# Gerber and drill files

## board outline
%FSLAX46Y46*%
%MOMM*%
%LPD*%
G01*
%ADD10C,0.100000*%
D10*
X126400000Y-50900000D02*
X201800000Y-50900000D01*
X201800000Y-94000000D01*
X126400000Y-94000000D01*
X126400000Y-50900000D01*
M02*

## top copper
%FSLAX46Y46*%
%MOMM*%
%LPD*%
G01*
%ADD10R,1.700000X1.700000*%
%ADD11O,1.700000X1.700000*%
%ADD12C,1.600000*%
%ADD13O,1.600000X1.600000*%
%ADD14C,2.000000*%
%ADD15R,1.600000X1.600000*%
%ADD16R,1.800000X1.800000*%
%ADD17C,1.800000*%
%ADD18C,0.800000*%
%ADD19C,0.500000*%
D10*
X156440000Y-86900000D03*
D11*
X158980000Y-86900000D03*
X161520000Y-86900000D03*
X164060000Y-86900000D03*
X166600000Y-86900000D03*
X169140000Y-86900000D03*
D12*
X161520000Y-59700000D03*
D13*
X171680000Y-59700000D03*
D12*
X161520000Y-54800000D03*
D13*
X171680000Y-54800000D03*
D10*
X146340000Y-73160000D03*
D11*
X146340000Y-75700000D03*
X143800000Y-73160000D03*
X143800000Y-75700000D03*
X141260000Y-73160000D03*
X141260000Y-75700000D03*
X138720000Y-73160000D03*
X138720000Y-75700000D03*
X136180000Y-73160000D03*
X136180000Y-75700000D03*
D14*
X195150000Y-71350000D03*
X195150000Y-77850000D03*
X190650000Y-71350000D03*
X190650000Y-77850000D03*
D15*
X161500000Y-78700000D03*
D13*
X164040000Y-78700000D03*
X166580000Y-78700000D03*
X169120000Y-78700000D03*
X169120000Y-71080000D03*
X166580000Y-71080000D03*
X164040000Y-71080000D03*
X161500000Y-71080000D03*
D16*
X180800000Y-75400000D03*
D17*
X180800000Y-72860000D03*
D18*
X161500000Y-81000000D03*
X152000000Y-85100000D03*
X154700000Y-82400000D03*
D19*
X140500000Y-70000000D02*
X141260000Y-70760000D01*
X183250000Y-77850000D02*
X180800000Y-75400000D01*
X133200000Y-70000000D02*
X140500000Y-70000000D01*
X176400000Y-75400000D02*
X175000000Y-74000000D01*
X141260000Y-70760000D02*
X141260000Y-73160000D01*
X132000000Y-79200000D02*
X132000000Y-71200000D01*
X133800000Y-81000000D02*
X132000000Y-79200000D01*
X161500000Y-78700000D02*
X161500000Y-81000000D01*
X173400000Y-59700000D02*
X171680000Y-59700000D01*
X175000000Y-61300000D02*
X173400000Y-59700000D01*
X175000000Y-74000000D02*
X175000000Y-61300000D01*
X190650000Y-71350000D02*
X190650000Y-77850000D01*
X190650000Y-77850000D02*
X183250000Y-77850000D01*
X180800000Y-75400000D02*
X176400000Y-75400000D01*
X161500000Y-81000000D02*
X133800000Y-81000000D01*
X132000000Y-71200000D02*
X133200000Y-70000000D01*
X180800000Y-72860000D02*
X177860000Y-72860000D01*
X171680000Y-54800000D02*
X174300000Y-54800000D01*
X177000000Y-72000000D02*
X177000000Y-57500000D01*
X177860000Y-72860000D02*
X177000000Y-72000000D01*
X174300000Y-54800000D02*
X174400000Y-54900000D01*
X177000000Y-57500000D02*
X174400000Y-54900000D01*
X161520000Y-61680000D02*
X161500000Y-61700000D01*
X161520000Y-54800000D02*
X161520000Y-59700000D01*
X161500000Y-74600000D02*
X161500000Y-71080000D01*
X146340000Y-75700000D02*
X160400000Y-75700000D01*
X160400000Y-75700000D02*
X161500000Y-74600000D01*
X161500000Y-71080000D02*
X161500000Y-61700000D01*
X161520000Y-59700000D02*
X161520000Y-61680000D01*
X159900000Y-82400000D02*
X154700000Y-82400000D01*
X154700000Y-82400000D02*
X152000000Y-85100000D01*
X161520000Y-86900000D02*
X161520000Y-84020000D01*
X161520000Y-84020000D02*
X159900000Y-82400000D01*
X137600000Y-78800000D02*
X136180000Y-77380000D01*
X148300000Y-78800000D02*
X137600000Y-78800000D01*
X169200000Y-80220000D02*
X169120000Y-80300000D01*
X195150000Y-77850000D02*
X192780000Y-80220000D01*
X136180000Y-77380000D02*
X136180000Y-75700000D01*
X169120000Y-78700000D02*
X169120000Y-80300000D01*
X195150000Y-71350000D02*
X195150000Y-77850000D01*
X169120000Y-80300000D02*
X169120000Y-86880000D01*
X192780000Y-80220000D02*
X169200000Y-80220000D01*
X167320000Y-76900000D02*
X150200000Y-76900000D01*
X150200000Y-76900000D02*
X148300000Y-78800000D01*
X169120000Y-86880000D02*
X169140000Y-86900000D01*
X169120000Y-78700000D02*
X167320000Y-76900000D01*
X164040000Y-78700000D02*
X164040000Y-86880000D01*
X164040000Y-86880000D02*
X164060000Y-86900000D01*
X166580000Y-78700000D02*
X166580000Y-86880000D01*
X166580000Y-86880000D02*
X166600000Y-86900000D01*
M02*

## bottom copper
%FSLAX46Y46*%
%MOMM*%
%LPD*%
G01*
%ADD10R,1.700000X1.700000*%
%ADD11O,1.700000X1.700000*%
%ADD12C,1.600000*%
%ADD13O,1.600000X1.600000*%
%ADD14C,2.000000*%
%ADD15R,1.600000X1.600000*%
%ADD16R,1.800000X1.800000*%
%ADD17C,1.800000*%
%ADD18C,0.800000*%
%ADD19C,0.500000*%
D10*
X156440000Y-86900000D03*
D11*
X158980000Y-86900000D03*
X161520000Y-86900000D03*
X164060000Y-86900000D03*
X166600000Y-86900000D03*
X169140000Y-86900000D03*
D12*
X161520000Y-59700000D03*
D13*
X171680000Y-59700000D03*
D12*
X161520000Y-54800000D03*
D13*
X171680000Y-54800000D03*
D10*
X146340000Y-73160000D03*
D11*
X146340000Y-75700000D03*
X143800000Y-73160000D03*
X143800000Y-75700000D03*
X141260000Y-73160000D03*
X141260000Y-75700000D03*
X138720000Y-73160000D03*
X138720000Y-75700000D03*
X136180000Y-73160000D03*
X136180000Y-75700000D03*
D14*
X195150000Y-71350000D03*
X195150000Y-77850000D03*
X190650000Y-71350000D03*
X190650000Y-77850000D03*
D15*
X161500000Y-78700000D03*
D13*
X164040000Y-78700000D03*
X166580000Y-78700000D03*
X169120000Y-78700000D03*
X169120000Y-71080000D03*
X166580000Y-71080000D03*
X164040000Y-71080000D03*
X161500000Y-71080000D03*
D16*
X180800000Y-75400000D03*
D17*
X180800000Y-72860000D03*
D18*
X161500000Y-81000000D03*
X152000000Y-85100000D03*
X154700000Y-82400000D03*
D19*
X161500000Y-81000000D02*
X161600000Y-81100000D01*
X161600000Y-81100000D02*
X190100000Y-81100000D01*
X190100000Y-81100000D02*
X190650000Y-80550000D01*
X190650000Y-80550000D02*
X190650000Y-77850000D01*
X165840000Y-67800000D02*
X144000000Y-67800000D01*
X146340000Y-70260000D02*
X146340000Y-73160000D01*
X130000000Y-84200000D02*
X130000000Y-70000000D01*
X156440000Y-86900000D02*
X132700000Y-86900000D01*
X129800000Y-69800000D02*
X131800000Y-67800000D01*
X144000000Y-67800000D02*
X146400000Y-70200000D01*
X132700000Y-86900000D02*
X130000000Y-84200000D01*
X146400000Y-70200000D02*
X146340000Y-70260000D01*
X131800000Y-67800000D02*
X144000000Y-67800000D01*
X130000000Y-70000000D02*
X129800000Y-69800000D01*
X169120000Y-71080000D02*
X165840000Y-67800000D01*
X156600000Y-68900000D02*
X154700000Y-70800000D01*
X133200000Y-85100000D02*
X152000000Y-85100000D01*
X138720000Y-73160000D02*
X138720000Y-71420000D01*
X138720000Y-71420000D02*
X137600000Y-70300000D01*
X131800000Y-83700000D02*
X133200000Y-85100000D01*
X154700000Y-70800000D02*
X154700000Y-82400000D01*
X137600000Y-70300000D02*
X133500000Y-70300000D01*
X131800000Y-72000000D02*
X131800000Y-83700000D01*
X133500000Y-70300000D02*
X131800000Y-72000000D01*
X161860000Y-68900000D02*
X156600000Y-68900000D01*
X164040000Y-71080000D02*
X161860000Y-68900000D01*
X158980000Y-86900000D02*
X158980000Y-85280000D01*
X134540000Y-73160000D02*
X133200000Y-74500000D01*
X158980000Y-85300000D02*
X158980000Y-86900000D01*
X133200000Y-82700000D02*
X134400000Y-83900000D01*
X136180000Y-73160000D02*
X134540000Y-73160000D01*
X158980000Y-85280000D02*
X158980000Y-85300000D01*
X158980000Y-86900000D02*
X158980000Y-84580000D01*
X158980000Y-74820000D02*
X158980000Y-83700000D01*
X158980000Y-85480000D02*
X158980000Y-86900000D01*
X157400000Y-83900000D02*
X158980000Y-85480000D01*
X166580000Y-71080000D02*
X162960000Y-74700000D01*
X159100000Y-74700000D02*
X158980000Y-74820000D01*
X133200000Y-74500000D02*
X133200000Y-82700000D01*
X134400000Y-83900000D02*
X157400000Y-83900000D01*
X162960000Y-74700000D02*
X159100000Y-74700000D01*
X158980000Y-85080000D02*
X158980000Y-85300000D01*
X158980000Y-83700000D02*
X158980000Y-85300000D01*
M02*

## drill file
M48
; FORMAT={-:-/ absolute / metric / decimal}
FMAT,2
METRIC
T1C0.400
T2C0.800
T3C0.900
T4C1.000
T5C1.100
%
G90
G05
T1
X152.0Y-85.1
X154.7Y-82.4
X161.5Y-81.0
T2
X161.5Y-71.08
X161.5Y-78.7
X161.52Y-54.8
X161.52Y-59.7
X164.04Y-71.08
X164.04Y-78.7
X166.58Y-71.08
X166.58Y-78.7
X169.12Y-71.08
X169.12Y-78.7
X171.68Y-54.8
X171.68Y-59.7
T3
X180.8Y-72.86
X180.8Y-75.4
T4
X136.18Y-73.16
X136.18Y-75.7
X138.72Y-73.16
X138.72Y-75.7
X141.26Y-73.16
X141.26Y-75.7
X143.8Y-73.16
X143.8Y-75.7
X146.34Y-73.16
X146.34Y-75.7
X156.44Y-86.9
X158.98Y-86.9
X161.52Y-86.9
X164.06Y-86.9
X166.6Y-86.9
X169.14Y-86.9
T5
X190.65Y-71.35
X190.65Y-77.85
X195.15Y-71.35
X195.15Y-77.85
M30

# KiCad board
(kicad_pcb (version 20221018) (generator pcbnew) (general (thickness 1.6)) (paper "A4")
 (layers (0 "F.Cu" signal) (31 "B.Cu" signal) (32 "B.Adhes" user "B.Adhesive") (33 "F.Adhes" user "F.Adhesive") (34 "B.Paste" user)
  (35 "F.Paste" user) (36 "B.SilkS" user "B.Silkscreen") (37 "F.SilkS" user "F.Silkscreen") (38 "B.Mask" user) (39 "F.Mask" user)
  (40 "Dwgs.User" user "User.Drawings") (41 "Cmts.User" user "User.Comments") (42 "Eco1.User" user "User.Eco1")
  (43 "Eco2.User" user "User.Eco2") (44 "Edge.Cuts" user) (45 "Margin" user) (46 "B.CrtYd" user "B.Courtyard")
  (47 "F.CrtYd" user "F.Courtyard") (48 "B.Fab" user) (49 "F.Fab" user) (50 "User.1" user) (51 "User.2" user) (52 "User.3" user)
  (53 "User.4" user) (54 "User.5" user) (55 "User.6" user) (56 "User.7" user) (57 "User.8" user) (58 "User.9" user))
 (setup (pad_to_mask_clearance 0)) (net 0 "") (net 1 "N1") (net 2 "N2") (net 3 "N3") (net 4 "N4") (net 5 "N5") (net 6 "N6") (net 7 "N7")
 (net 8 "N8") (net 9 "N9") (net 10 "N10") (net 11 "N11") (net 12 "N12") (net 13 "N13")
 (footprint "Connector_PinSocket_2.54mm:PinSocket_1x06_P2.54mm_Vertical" (layer "F.Cu") (at 156.44 86.9 90)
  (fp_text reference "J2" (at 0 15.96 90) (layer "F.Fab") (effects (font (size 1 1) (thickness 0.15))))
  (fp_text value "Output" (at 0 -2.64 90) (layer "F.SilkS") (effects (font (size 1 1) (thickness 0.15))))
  (pad "1" thru_hole rect (at 0 0 90) (size 1.7 1.7) (drill 1) (layers "*.Cu" "*.Mask") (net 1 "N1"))
  (pad "2" thru_hole oval (at 0 2.54 90) (size 1.7 1.7) (drill 1) (layers "*.Cu" "*.Mask") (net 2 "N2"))
  (pad "3" thru_hole oval (at 0 5.08 90) (size 1.7 1.7) (drill 1) (layers "*.Cu" "*.Mask") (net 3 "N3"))
  (pad "4" thru_hole oval (at 0 7.62 90) (size 1.7 1.7) (drill 1) (layers "*.Cu" "*.Mask") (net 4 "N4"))
  (pad "5" thru_hole oval (at 0 10.16 90) (size 1.7 1.7) (drill 1) (layers "*.Cu" "*.Mask") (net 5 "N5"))
  (pad "6" thru_hole oval (at 0 12.7 90) (size 1.7 1.7) (drill 1) (layers "*.Cu" "*.Mask") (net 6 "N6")))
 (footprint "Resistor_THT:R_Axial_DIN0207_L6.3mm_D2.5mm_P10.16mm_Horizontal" (layer "F.Cu") (at 161.52 59.7)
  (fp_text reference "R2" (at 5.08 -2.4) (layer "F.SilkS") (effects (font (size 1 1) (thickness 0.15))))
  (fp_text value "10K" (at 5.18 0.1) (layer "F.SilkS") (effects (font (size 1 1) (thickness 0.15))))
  (pad "1" thru_hole circle (at 0 0) (size 1.6 1.6) (drill 0.8) (layers "*.Cu" "*.Mask") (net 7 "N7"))
  (pad "2" thru_hole oval (at 10.16 0) (size 1.6 1.6) (drill 0.8) (layers "*.Cu" "*.Mask") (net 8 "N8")))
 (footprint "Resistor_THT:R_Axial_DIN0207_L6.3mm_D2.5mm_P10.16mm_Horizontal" (layer "F.Cu") (at 161.52 54.8)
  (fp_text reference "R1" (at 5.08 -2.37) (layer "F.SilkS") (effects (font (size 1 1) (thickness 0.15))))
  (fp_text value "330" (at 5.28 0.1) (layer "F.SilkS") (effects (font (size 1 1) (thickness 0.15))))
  (pad "1" thru_hole circle (at 0 0) (size 1.6 1.6) (drill 0.8) (layers "*.Cu" "*.Mask") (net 7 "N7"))
  (pad "2" thru_hole oval (at 10.16 0) (size 1.6 1.6) (drill 0.8) (layers "*.Cu" "*.Mask") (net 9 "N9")))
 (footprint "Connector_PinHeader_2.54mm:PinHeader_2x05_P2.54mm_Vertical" (layer "F.Cu") (at 146.34 73.16 -90)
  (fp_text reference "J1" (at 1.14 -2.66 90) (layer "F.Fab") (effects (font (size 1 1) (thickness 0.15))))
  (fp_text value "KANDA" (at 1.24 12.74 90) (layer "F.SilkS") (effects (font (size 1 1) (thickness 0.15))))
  (pad "1" thru_hole rect (at 0 0 270) (size 1.7 1.7) (drill 1) (layers "*.Cu" "*.Mask") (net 1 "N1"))
  (pad "2" thru_hole oval (at 2.54 0 270) (size 1.7 1.7) (drill 1) (layers "*.Cu" "*.Mask") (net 7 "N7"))
  (pad "3" thru_hole oval (at 0 2.54 270) (size 1.7 1.7) (drill 1) (layers "*.Cu" "*.Mask") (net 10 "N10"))
  (pad "4" thru_hole oval (at 2.54 2.54 270) (size 1.7 1.7) (drill 1) (layers "*.Cu" "*.Mask") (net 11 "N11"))
  (pad "5" thru_hole oval (at 0 5.08 270) (size 1.7 1.7) (drill 1) (layers "*.Cu" "*.Mask") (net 8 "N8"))
  (pad "6" thru_hole oval (at 2.54 5.08 270) (size 1.7 1.7) (drill 1) (layers "*.Cu" "*.Mask") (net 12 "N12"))
  (pad "7" thru_hole oval (at 0 7.62 270) (size 1.7 1.7) (drill 1) (layers "*.Cu" "*.Mask") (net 3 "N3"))
  (pad "8" thru_hole oval (at 2.54 7.62 270) (size 1.7 1.7) (drill 1) (layers "*.Cu" "*.Mask") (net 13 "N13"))
  (pad "9" thru_hole oval (at 0 10.16 270) (size 1.7 1.7) (drill 1) (layers "*.Cu" "*.Mask") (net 2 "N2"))
  (pad "10" thru_hole oval (at 2.54 10.16 270) (size 1.7 1.7) (drill 1) (layers "*.Cu" "*.Mask") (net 6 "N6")))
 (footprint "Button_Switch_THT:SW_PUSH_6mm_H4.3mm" (layer "F.Cu") (at 195.15 71.35 -90)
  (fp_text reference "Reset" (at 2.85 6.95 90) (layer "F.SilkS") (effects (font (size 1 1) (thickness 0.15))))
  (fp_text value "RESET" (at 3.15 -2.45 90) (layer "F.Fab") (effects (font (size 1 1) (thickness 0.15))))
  (pad "1" thru_hole circle (at 0 0) (size 2 2) (drill 1.1) (layers "*.Cu" "*.Mask") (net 6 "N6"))
  (pad "1" thru_hole circle (at 6.5 0) (size 2 2) (drill 1.1) (layers "*.Cu" "*.Mask") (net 6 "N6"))
  (pad "2" thru_hole circle (at 0 4.5) (size 2 2) (drill 1.1) (layers "*.Cu" "*.Mask") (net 8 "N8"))
  (pad "2" thru_hole circle (at 6.5 4.5) (size 2 2) (drill 1.1) (layers "*.Cu" "*.Mask") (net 8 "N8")))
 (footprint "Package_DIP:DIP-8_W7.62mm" (layer "F.Cu") (at 161.5 78.7 90)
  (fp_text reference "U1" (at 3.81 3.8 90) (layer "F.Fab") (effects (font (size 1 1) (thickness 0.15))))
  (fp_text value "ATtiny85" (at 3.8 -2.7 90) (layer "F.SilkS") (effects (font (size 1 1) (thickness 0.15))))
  (pad "1" thru_hole rect (at 0 0 90) (size 1.6 1.6) (drill 0.8) (layers "*.Cu" "*.Mask") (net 8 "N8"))
  (pad "2" thru_hole oval (at 0 2.54 90) (size 1.6 1.6) (drill 0.8) (layers "*.Cu" "*.Mask") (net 4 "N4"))
  (pad "3" thru_hole oval (at 0 5.08 90) (size 1.6 1.6) (drill 0.8) (layers "*.Cu" "*.Mask") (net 5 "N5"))
  (pad "4" thru_hole oval (at 0 7.62 90) (size 1.6 1.6) (drill 0.8) (layers "*.Cu" "*.Mask") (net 6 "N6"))
  (pad "5" thru_hole oval (at 7.62 7.62 90) (size 1.6 1.6) (drill 0.8) (layers "*.Cu" "*.Mask") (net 1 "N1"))
  (pad "6" thru_hole oval (at 7.62 5.08 90) (size 1.6 1.6) (drill 0.8) (layers "*.Cu" "*.Mask") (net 2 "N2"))
  (pad "7" thru_hole oval (at 7.62 2.54 90) (size 1.6 1.6) (drill 0.8) (layers "*.Cu" "*.Mask") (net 3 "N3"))
  (pad "8" thru_hole oval (at 7.62 0 90) (size 1.6 1.6) (drill 0.8) (layers "*.Cu" "*.Mask") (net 7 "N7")))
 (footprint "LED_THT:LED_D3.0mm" (layer "F.Cu") (at 180.8 75.4 90)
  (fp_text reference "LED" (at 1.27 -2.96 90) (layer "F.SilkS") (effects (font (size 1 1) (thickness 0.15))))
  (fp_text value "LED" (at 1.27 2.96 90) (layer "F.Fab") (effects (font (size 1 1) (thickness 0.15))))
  (pad "1" thru_hole rect (at 0 0 90) (size 1.8 1.8) (drill 0.9) (layers "*.Cu" "*.Mask") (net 8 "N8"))
  (pad "2" thru_hole circle (at 2.54 0 90) (size 1.8 1.8) (drill 0.9) (layers "*.Cu" "*.Mask") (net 9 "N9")))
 (gr_rect (start 126.4 50.9) (end 201.8 94) (stroke (width 0.1) (type default)) (fill none) (layer "Edge.Cuts"))
 (segment (start 140.5 70) (end 141.26 70.76) (width 0.5) (layer "F.Cu") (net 8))
 (segment (start 183.25 77.85) (end 180.8 75.4) (width 0.5) (layer "F.Cu") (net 8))
 (segment (start 133.2 70) (end 140.5 70) (width 0.5) (layer "F.Cu") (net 8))
 (segment (start 176.4 75.4) (end 175 74) (width 0.5) (layer "F.Cu") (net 8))
 (segment (start 141.26 70.76) (end 141.26 73.16) (width 0.5) (layer "F.Cu") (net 8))
 (segment (start 132 79.2) (end 132 71.2) (width 0.5) (layer "F.Cu") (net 8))
 (segment (start 133.8 81) (end 132 79.2) (width 0.5) (layer "F.Cu") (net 8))
 (segment (start 161.5 78.7) (end 161.5 81) (width 0.5) (layer "F.Cu") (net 8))
 (segment (start 173.4 59.7) (end 171.68 59.7) (width 0.5) (layer "F.Cu") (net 8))
 (segment (start 175 61.3) (end 173.4 59.7) (width 0.5) (layer "F.Cu") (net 8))
 (segment (start 175 74) (end 175 61.3) (width 0.5) (layer "F.Cu") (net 8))
 (segment (start 190.65 71.35) (end 190.65 77.85) (width 0.5) (layer "F.Cu") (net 8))
 (segment (start 190.65 77.85) (end 183.25 77.85) (width 0.5) (layer "F.Cu") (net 8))
 (segment (start 180.8 75.4) (end 176.4 75.4) (width 0.5) (layer "F.Cu") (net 8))
 (segment (start 161.5 81) (end 133.8 81) (width 0.5) (layer "F.Cu") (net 8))
 (segment (start 132 71.2) (end 133.2 70) (width 0.5) (layer "F.Cu") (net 8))
 (via (at 161.5 81) (size 0.8) (drill 0.4) (layers "F.Cu" "B.Cu") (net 8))
 (segment (start 161.5 81) (end 161.6 81.1) (width 0.5) (layer "B.Cu") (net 8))
 (segment (start 161.6 81.1) (end 190.1 81.1) (width 0.5) (layer "B.Cu") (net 8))
 (segment (start 190.1 81.1) (end 190.65 80.55) (width 0.5) (layer "B.Cu") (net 8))
 (segment (start 190.65 80.55) (end 190.65 77.85) (width 0.5) (layer "B.Cu") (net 8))
 (segment (start 180.8 72.86) (end 177.86 72.86) (width 0.5) (layer "F.Cu") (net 9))
 (segment (start 171.68 54.8) (end 174.3 54.8) (width 0.5) (layer "F.Cu") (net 9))
 (segment (start 177 72) (end 177 57.5) (width 0.5) (layer "F.Cu") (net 9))
 (segment (start 177.86 72.86) (end 177 72) (width 0.5) (layer "F.Cu") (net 9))
 (segment (start 174.3 54.8) (end 174.4 54.9) (width 0.5) (layer "F.Cu") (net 9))
 (segment (start 177 57.5) (end 174.4 54.9) (width 0.5) (layer "F.Cu") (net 9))
 (segment (start 165.84 67.8) (end 144 67.8) (width 0.5) (layer "B.Cu") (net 1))
 (segment (start 146.34 70.26) (end 146.34 73.16) (width 0.5) (layer "B.Cu") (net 1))
 (segment (start 130 84.2) (end 130 70) (width 0.5) (layer "B.Cu") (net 1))
 (segment (start 156.44 86.9) (end 132.7 86.9) (width 0.5) (layer "B.Cu") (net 1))
 (segment (start 129.8 69.8) (end 131.8 67.8) (width 0.5) (layer "B.Cu") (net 1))
 (segment (start 144 67.8) (end 146.4 70.2) (width 0.5) (layer "B.Cu") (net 1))
 (segment (start 132.7 86.9) (end 130 84.2) (width 0.5) (layer "B.Cu") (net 1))
 (segment (start 146.4 70.2) (end 146.34 70.26) (width 0.5) (layer "B.Cu") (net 1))
 (segment (start 131.8 67.8) (end 144 67.8) (width 0.5) (layer "B.Cu") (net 1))
 (segment (start 130 70) (end 129.8 69.8) (width 0.5) (layer "B.Cu") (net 1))
 (segment (start 169.12 71.08) (end 165.84 67.8) (width 0.5) (layer "B.Cu") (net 1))
 (segment (start 161.52 61.68) (end 161.5 61.7) (width 0.5) (layer "F.Cu") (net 7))
 (segment (start 161.52 54.8) (end 161.52 59.7) (width 0.5) (layer "F.Cu") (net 7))
 (segment (start 161.5 74.6) (end 161.5 71.08) (width 0.5) (layer "F.Cu") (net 7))
 (segment (start 146.34 75.7) (end 160.4 75.7) (width 0.5) (layer "F.Cu") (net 7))
 (segment (start 160.4 75.7) (end 161.5 74.6) (width 0.5) (layer "F.Cu") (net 7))
 (segment (start 161.5 71.08) (end 161.5 61.7) (width 0.5) (layer "F.Cu") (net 7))
 (segment (start 161.52 59.7) (end 161.52 61.68) (width 0.5) (layer "F.Cu") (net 7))
 (segment (start 159.9 82.4) (end 154.7 82.4) (width 0.5) (layer "F.Cu") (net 3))
 (segment (start 154.7 82.4) (end 152 85.1) (width 0.5) (layer "F.Cu") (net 3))
 (segment (start 161.52 86.9) (end 161.52 84.02) (width 0.5) (layer "F.Cu") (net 3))
 (segment (start 161.52 84.02) (end 159.9 82.4) (width 0.5) (layer "F.Cu") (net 3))
 (via (at 152 85.1) (size 0.8) (drill 0.4) (layers "F.Cu" "B.Cu") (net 3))
 (via (at 154.7 82.4) (size 0.8) (drill 0.4) (layers "F.Cu" "B.Cu") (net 3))
 (segment (start 156.6 68.9) (end 154.7 70.8) (width 0.5) (layer "B.Cu") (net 3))
 (segment (start 133.2 85.1) (end 152 85.1) (width 0.5) (layer "B.Cu") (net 3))
 (segment (start 138.72 73.16) (end 138.72 71.42) (width 0.5) (layer "B.Cu") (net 3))
 (segment (start 138.72 71.42) (end 137.6 70.3) (width 0.5) (layer "B.Cu") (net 3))
 (segment (start 131.8 83.7) (end 133.2 85.1) (width 0.5) (layer "B.Cu") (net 3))
 (segment (start 154.7 70.8) (end 154.7 82.4) (width 0.5) (layer "B.Cu") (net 3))
 (segment (start 137.6 70.3) (end 133.5 70.3) (width 0.5) (layer "B.Cu") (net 3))
 (segment (start 131.8 72) (end 131.8 83.7) (width 0.5) (layer "B.Cu") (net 3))
 (segment (start 133.5 70.3) (end 131.8 72) (width 0.5) (layer "B.Cu") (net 3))
 (segment (start 161.86 68.9) (end 156.6 68.9) (width 0.5) (layer "B.Cu") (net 3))
 (segment (start 164.04 71.08) (end 161.86 68.9) (width 0.5) (layer "B.Cu") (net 3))
 (segment (start 158.98 86.9) (end 158.98 85.28) (width 0.5) (layer "B.Cu") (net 2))
 (segment (start 134.54 73.16) (end 133.2 74.5) (width 0.5) (layer "B.Cu") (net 2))
 (segment (start 158.98 85.3) (end 158.98 86.9) (width 0.5) (layer "B.Cu") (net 2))
 (segment (start 133.2 82.7) (end 134.4 83.9) (width 0.5) (layer "B.Cu") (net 2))
 (segment (start 136.18 73.16) (end 134.54 73.16) (width 0.5) (layer "B.Cu") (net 2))
 (segment (start 158.98 85.28) (end 158.98 85.3) (width 0.5) (layer "B.Cu") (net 2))
 (segment (start 158.98 86.9) (end 158.98 84.58) (width 0.5) (layer "B.Cu") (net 2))
 (segment (start 158.98 74.82) (end 158.98 83.7) (width 0.5) (layer "B.Cu") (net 2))
 (segment (start 158.98 85.48) (end 158.98 86.9) (width 0.5) (layer "B.Cu") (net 2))
 (segment (start 157.4 83.9) (end 158.98 85.48) (width 0.5) (layer "B.Cu") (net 2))
 (segment (start 166.58 71.08) (end 162.96 74.7) (width 0.5) (layer "B.Cu") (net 2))
 (segment (start 159.1 74.7) (end 158.98 74.82) (width 0.5) (layer "B.Cu") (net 2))
 (segment (start 133.2 74.5) (end 133.2 82.7) (width 0.5) (layer "B.Cu") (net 2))
 (segment (start 134.4 83.9) (end 157.4 83.9) (width 0.5) (layer "B.Cu") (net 2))
 (segment (start 162.96 74.7) (end 159.1 74.7) (width 0.5) (layer "B.Cu") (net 2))
 (segment (start 158.98 85.08) (end 158.98 85.3) (width 0.5) (layer "B.Cu") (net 2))
 (segment (start 158.98 83.7) (end 158.98 85.3) (width 0.5) (layer "B.Cu") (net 2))
 (segment (start 137.6 78.8) (end 136.18 77.38) (width 0.5) (layer "F.Cu") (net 6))
 (segment (start 148.3 78.8) (end 137.6 78.8) (width 0.5) (layer "F.Cu") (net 6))
 (segment (start 169.2 80.22) (end 169.12 80.3) (width 0.5) (layer "F.Cu") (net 6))
 (segment (start 195.15 77.85) (end 192.78 80.22) (width 0.5) (layer "F.Cu") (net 6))
 (segment (start 136.18 77.38) (end 136.18 75.7) (width 0.5) (layer "F.Cu") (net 6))
 (segment (start 169.12 78.7) (end 169.12 80.3) (width 0.5) (layer "F.Cu") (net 6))
 (segment (start 195.15 71.35) (end 195.15 77.85) (width 0.5) (layer "F.Cu") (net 6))
 (segment (start 169.12 80.3) (end 169.12 86.88) (width 0.5) (layer "F.Cu") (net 6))
 (segment (start 192.78 80.22) (end 169.2 80.22) (width 0.5) (layer "F.Cu") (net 6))
 (segment (start 167.32 76.9) (end 150.2 76.9) (width 0.5) (layer "F.Cu") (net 6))
 (segment (start 150.2 76.9) (end 148.3 78.8) (width 0.5) (layer "F.Cu") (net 6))
 (segment (start 169.12 86.88) (end 169.14 86.9) (width 0.5) (layer "F.Cu") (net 6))
 (segment (start 169.12 78.7) (end 167.32 76.9) (width 0.5) (layer "F.Cu") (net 6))
 (segment (start 164.04 78.7) (end 164.04 86.88) (width 0.5) (layer "F.Cu") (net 4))
 (segment (start 164.04 86.88) (end 164.06 86.9) (width 0.5) (layer "F.Cu") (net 4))
 (segment (start 166.58 78.7) (end 166.58 86.88) (width 0.5) (layer "F.Cu") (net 5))
 (segment (start 166.58 86.88) (end 166.6 86.9) (width 0.5) (layer "F.Cu") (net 5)))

